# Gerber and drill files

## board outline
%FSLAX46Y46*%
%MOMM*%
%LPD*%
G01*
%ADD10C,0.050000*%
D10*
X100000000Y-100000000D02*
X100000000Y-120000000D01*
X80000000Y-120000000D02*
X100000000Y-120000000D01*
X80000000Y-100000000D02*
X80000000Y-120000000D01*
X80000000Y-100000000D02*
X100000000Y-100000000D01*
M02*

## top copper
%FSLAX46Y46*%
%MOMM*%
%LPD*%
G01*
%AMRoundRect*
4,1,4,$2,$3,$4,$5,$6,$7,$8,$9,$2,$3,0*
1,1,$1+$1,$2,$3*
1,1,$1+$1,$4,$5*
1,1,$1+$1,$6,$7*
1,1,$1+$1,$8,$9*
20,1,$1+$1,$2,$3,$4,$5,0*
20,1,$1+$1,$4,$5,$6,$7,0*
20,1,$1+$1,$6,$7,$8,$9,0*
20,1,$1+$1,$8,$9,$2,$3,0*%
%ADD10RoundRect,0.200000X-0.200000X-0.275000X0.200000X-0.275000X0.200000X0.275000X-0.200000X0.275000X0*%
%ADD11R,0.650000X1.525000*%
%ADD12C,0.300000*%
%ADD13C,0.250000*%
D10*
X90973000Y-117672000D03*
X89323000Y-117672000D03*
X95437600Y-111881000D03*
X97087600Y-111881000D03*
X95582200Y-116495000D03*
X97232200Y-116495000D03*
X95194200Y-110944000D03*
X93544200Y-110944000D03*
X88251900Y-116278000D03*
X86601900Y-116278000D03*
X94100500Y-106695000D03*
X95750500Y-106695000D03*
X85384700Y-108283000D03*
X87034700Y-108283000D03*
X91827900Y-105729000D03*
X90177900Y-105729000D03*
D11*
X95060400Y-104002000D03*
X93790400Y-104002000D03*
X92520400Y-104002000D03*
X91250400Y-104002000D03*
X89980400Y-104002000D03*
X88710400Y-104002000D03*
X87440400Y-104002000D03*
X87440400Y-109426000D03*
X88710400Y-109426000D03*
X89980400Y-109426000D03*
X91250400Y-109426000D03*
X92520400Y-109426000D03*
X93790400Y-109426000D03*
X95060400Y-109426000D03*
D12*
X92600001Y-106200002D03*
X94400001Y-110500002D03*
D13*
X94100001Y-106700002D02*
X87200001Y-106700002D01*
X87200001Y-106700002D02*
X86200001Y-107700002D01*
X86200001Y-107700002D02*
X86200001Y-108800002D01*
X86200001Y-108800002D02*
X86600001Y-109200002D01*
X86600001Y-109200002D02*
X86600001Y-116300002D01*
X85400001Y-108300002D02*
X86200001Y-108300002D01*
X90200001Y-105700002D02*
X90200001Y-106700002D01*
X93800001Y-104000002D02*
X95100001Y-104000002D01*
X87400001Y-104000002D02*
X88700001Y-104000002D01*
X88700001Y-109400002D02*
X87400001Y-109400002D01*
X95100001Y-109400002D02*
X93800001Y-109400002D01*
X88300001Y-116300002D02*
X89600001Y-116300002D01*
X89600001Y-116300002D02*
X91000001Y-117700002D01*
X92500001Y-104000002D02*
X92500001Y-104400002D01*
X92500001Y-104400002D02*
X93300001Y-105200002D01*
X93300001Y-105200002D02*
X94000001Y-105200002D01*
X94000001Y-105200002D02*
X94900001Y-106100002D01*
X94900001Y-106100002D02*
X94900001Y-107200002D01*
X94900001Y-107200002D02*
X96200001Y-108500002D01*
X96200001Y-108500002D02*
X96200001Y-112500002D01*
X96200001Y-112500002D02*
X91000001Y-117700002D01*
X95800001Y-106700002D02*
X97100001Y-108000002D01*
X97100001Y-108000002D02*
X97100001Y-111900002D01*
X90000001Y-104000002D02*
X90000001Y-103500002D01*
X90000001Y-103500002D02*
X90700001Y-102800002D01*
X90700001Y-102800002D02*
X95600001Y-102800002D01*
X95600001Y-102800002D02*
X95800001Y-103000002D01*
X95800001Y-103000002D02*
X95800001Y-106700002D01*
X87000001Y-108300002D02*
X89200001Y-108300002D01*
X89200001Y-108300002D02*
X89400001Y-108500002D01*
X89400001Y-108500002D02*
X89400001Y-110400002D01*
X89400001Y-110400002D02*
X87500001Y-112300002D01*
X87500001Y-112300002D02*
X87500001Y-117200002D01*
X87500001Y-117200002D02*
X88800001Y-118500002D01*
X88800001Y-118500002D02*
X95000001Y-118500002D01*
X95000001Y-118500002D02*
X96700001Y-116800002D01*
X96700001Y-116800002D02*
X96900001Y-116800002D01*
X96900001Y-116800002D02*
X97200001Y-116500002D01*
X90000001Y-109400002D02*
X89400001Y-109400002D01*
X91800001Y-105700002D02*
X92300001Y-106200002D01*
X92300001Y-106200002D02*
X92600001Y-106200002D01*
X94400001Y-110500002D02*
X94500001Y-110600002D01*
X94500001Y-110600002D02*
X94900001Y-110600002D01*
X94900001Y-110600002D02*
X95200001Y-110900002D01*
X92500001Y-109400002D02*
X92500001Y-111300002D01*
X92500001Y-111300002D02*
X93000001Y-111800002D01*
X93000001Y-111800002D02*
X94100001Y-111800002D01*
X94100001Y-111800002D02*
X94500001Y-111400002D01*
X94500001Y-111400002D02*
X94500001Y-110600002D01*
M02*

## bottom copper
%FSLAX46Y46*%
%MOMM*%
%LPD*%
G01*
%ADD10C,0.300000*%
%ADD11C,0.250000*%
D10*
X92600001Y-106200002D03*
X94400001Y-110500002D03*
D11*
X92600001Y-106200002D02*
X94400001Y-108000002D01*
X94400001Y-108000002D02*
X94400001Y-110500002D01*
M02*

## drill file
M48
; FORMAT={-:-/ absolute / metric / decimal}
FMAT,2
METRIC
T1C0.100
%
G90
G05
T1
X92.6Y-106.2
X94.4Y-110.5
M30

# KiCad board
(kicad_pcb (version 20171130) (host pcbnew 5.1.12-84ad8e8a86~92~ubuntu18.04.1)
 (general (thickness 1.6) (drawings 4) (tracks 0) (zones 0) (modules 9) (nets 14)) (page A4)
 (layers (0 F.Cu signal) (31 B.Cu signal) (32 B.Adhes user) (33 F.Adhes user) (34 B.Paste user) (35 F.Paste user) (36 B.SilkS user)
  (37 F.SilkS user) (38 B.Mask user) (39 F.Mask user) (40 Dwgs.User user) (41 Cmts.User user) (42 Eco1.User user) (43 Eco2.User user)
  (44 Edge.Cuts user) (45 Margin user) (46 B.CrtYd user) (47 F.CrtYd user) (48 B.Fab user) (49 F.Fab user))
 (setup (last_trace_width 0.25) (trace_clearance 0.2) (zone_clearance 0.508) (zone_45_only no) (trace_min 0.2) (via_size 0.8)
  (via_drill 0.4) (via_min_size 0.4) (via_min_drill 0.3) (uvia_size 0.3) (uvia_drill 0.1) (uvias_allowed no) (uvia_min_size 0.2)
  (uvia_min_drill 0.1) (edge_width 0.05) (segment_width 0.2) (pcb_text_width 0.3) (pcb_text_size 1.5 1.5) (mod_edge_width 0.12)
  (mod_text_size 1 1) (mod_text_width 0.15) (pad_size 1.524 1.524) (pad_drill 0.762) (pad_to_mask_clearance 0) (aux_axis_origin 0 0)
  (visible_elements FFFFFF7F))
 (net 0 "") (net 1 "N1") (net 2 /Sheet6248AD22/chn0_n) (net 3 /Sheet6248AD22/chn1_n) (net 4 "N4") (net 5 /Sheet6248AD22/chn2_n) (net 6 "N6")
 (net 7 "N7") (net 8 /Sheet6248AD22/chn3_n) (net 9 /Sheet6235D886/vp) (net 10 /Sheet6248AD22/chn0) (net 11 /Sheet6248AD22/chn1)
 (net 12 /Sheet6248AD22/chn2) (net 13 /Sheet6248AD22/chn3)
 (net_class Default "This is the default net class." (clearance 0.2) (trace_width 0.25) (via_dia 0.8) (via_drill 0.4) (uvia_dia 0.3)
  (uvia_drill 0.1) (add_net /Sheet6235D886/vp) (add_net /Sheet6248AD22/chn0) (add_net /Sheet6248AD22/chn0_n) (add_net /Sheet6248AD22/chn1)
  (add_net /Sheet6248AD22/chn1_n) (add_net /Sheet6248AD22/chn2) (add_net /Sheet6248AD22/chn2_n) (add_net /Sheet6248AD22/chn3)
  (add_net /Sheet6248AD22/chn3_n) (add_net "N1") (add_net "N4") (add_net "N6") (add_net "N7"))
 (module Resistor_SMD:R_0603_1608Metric (layer F.Cu) (at 90.148000 117.672000)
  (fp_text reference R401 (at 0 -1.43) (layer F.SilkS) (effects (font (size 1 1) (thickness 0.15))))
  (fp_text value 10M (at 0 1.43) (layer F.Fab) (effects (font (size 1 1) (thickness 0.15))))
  (pad 2 smd roundrect (at 0.825 0) (size 0.8 0.95) (layers F.Cu F.Mask F.Paste) (roundrect_rratio 0.25) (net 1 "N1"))
  (pad 1 smd roundrect (at -0.825 0) (size 0.8 0.95) (layers F.Cu F.Mask F.Paste) (roundrect_rratio 0.25) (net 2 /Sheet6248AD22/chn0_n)))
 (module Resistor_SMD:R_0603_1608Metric (layer F.Cu) (at 96.262600 111.881000)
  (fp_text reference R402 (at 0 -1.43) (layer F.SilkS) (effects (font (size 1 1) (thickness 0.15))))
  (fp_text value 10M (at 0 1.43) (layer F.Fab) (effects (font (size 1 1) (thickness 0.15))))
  (pad 1 smd roundrect (at -0.825 0) (size 0.8 0.95) (layers F.Cu F.Mask F.Paste) (roundrect_rratio 0.25) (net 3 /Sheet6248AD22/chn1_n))
  (pad 2 smd roundrect (at 0.825 0) (size 0.8 0.95) (layers F.Cu F.Mask F.Paste) (roundrect_rratio 0.25) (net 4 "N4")))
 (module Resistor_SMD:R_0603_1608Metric (layer F.Cu) (at 96.407200 116.495000)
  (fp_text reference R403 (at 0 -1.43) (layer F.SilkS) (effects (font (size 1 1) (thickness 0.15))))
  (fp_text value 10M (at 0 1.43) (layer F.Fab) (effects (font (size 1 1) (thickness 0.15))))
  (pad 1 smd roundrect (at -0.825 0) (size 0.8 0.95) (layers F.Cu F.Mask F.Paste) (roundrect_rratio 0.25) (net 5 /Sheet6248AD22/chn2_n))
  (pad 2 smd roundrect (at 0.825 0) (size 0.8 0.95) (layers F.Cu F.Mask F.Paste) (roundrect_rratio 0.25) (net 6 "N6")))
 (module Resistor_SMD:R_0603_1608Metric (layer F.Cu) (at 94.369200 110.944000)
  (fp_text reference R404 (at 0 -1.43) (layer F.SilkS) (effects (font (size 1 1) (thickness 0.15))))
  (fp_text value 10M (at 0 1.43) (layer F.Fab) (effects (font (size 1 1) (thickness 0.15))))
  (pad 2 smd roundrect (at 0.825 0) (size 0.8 0.95) (layers F.Cu F.Mask F.Paste) (roundrect_rratio 0.25) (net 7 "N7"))
  (pad 1 smd roundrect (at -0.825 0) (size 0.8 0.95) (layers F.Cu F.Mask F.Paste) (roundrect_rratio 0.25) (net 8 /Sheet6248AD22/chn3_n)))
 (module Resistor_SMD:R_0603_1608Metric (layer F.Cu) (at 87.426900 116.278000)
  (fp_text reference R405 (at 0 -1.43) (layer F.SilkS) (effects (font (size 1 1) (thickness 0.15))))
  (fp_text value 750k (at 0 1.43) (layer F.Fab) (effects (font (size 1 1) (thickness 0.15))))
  (pad 2 smd roundrect (at 0.825 0) (size 0.8 0.95) (layers F.Cu F.Mask F.Paste) (roundrect_rratio 0.25) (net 1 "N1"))
  (pad 1 smd roundrect (at -0.825 0) (size 0.8 0.95) (layers F.Cu F.Mask F.Paste) (roundrect_rratio 0.25) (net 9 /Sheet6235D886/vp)))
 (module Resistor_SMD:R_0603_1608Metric (layer F.Cu) (at 94.925500 106.695000)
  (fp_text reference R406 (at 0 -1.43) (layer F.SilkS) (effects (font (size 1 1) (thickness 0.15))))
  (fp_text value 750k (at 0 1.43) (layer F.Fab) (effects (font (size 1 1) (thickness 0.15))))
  (pad 1 smd roundrect (at -0.825 0) (size 0.8 0.95) (layers F.Cu F.Mask F.Paste) (roundrect_rratio 0.25) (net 9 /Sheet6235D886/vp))
  (pad 2 smd roundrect (at 0.825 0) (size 0.8 0.95) (layers F.Cu F.Mask F.Paste) (roundrect_rratio 0.25) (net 4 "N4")))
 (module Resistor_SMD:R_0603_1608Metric (layer F.Cu) (at 86.209700 108.283000)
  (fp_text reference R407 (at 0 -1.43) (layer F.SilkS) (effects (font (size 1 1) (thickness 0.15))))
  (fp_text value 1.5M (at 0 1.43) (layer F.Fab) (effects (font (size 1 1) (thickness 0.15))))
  (pad 1 smd roundrect (at -0.825 0) (size 0.8 0.95) (layers F.Cu F.Mask F.Paste) (roundrect_rratio 0.25) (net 9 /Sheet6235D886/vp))
  (pad 2 smd roundrect (at 0.825 0) (size 0.8 0.95) (layers F.Cu F.Mask F.Paste) (roundrect_rratio 0.25) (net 6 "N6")))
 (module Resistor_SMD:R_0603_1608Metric (layer F.Cu) (at 91.002900 105.729000)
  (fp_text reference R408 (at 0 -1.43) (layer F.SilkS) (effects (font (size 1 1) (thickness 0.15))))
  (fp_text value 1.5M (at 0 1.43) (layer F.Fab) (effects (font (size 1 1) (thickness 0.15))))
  (pad 2 smd roundrect (at 0.825 0) (size 0.8 0.95) (layers F.Cu F.Mask F.Paste) (roundrect_rratio 0.25) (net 7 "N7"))
  (pad 1 smd roundrect (at -0.825 0) (size 0.8 0.95) (layers F.Cu F.Mask F.Paste) (roundrect_rratio 0.25) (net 9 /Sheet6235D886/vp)))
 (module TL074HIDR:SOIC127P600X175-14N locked (layer F.Cu) (at 91.250400 106.714000 270.000000)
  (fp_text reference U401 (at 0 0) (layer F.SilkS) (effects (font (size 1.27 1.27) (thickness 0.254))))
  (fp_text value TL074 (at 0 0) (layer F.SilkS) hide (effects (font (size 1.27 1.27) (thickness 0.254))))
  (pad 1 smd rect (at -2.712 -3.81) (size 0.65 1.525) (layers F.Cu F.Mask F.Paste) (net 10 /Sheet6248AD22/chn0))
  (pad 2 smd rect (at -2.712 -2.54) (size 0.65 1.525) (layers F.Cu F.Mask F.Paste) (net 10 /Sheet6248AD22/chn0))
  (pad 3 smd rect (at -2.712 -1.27) (size 0.65 1.525) (layers F.Cu F.Mask F.Paste) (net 1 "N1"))
  (pad 4 smd rect (at -2.712 0) (size 0.65 1.525) (layers F.Cu F.Mask F.Paste))
  (pad 5 smd rect (at -2.712 1.27) (size 0.65 1.525) (layers F.Cu F.Mask F.Paste) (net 4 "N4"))
  (pad 6 smd rect (at -2.712 2.54) (size 0.65 1.525) (layers F.Cu F.Mask F.Paste) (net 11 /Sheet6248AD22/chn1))
  (pad 7 smd rect (at -2.712 3.81) (size 0.65 1.525) (layers F.Cu F.Mask F.Paste) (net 11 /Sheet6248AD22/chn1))
  (pad 8 smd rect (at 2.712 3.81) (size 0.65 1.525) (layers F.Cu F.Mask F.Paste) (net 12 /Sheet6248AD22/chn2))
  (pad 9 smd rect (at 2.712 2.54) (size 0.65 1.525) (layers F.Cu F.Mask F.Paste) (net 12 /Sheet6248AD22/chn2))
  (pad 10 smd rect (at 2.712 1.27) (size 0.65 1.525) (layers F.Cu F.Mask F.Paste) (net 6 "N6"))
  (pad 11 smd rect (at 2.712 0) (size 0.65 1.525) (layers F.Cu F.Mask F.Paste))
  (pad 12 smd rect (at 2.712 -1.27) (size 0.65 1.525) (layers F.Cu F.Mask F.Paste) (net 7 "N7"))
  (pad 13 smd rect (at 2.712 -2.54) (size 0.65 1.525) (layers F.Cu F.Mask F.Paste) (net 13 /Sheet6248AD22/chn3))
  (pad 14 smd rect (at 2.712 -3.81) (size 0.65 1.525) (layers F.Cu F.Mask F.Paste) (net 13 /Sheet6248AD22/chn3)))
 (gr_line (start 100 100) (end 100 120) (layer Edge.Cuts) (width 0.05))
 (gr_line (start 80 120) (end 100 120) (layer Edge.Cuts) (width 0.05))
 (gr_line (start 80 100) (end 80 120) (layer Edge.Cuts) (width 0.05))
 (gr_line (start 80 100) (end 100 100) (layer Edge.Cuts) (width 0.05))
 (segment (start 94.100001 106.700002) (end 87.200001 106.700002) (width 0.250000) (layer F.Cu) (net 9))
 (segment (start 87.200001 106.700002) (end 86.200001 107.700002) (width 0.250000) (layer F.Cu) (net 9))
 (segment (start 86.200001 107.700002) (end 86.200001 108.800002) (width 0.250000) (layer F.Cu) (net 9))
 (segment (start 86.200001 108.800002) (end 86.600001 109.200002) (width 0.250000) (layer F.Cu) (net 9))
 (segment (start 86.600001 109.200002) (end 86.600001 116.300002) (width 0.250000) (layer F.Cu) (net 9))
 (segment (start 85.400001 108.300002) (end 86.200001 108.300002) (width 0.250000) (layer F.Cu) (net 9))
 (segment (start 90.200001 105.700002) (end 90.200001 106.700002) (width 0.250000) (layer F.Cu) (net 9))
 (segment (start 93.800001 104.000002) (end 95.100001 104.000002) (width 0.250000) (layer F.Cu) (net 10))
 (segment (start 87.400001 104.000002) (end 88.700001 104.000002) (width 0.250000) (layer F.Cu) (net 11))
 (segment (start 88.700001 109.400002) (end 87.400001 109.400002) (width 0.250000) (layer F.Cu) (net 12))
 (segment (start 95.100001 109.400002) (end 93.800001 109.400002) (width 0.250000) (layer F.Cu) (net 13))
 (segment (start 88.300001 116.300002) (end 89.600001 116.300002) (width 0.250000) (layer F.Cu) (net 1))
 (segment (start 89.600001 116.300002) (end 91.000001 117.700002) (width 0.250000) (layer F.Cu) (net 1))
 (segment (start 92.500001 104.000002) (end 92.500001 104.400002) (width 0.250000) (layer F.Cu) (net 1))
 (segment (start 92.500001 104.400002) (end 93.300001 105.200002) (width 0.250000) (layer F.Cu) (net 1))
 (segment (start 93.300001 105.200002) (end 94.000001 105.200002) (width 0.250000) (layer F.Cu) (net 1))
 (segment (start 94.000001 105.200002) (end 94.900001 106.100002) (width 0.250000) (layer F.Cu) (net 1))
 (segment (start 94.900001 106.100002) (end 94.900001 107.200002) (width 0.250000) (layer F.Cu) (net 1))
 (segment (start 94.900001 107.200002) (end 96.200001 108.500002) (width 0.250000) (layer F.Cu) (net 1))
 (segment (start 96.200001 108.500002) (end 96.200001 112.500002) (width 0.250000) (layer F.Cu) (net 1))
 (segment (start 96.200001 112.500002) (end 91.000001 117.700002) (width 0.250000) (layer F.Cu) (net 1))
 (segment (start 95.800001 106.700002) (end 97.100001 108.000002) (width 0.250000) (layer F.Cu) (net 4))
 (segment (start 97.100001 108.000002) (end 97.100001 111.900002) (width 0.250000) (layer F.Cu) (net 4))
 (segment (start 90.000001 104.000002) (end 90.000001 103.500002) (width 0.250000) (layer F.Cu) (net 4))
 (segment (start 90.000001 103.500002) (end 90.700001 102.800002) (width 0.250000) (layer F.Cu) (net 4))
 (segment (start 90.700001 102.800002) (end 95.600001 102.800002) (width 0.250000) (layer F.Cu) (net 4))
 (segment (start 95.600001 102.800002) (end 95.800001 103.000002) (width 0.250000) (layer F.Cu) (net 4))
 (segment (start 95.800001 103.000002) (end 95.800001 106.700002) (width 0.250000) (layer F.Cu) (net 4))
 (segment (start 87.000001 108.300002) (end 89.200001 108.300002) (width 0.250000) (layer F.Cu) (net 6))
 (segment (start 89.200001 108.300002) (end 89.400001 108.500002) (width 0.250000) (layer F.Cu) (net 6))
 (segment (start 89.400001 108.500002) (end 89.400001 110.400002) (width 0.250000) (layer F.Cu) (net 6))
 (segment (start 89.400001 110.400002) (end 87.500001 112.300002) (width 0.250000) (layer F.Cu) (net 6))
 (segment (start 87.500001 112.300002) (end 87.500001 117.200002) (width 0.250000) (layer F.Cu) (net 6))
 (segment (start 87.500001 117.200002) (end 88.800001 118.500002) (width 0.250000) (layer F.Cu) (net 6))
 (segment (start 88.800001 118.500002) (end 95.000001 118.500002) (width 0.250000) (layer F.Cu) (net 6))
 (segment (start 95.000001 118.500002) (end 96.700001 116.800002) (width 0.250000) (layer F.Cu) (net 6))
 (segment (start 96.700001 116.800002) (end 96.900001 116.800002) (width 0.250000) (layer F.Cu) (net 6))
 (segment (start 96.900001 116.800002) (end 97.200001 116.500002) (width 0.250000) (layer F.Cu) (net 6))
 (segment (start 90.000001 109.400002) (end 89.400001 109.400002) (width 0.250000) (layer F.Cu) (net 6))
 (segment (start 91.800001 105.700002) (end 92.300001 106.200002) (width 0.250000) (layer F.Cu) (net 7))
 (segment (start 92.300001 106.200002) (end 92.600001 106.200002) (width 0.250000) (layer F.Cu) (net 7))
 (segment (start 92.600001 106.200002) (end 94.400001 108.000002) (width 0.250000) (layer B.Cu) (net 7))
 (segment (start 94.400001 108.000002) (end 94.400001 110.500002) (width 0.250000) (layer B.Cu) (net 7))
 (segment (start 94.400001 110.500002) (end 94.500001 110.600002) (width 0.250000) (layer F.Cu) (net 7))
 (segment (start 94.500001 110.600002) (end 94.900001 110.600002) (width 0.250000) (layer F.Cu) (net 7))
 (segment (start 94.900001 110.600002) (end 95.200001 110.900002) (width 0.250000) (layer F.Cu) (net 7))
 (segment (start 92.500001 109.400002) (end 92.500001 111.300002) (width 0.250000) (layer F.Cu) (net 7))
 (segment (start 92.500001 111.300002) (end 93.000001 111.800002) (width 0.250000) (layer F.Cu) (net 7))
 (segment (start 93.000001 111.800002) (end 94.100001 111.800002) (width 0.250000) (layer F.Cu) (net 7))
 (segment (start 94.100001 111.800002) (end 94.500001 111.400002) (width 0.250000) (layer F.Cu) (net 7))
 (segment (start 94.500001 111.400002) (end 94.500001 110.600002) (width 0.250000) (layer F.Cu) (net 7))
 (via micro (at 92.600001 106.200002) (size 0.300000) (drill 0.100000) (layers F.Cu B.Cu) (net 7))
 (via micro (at 94.400001 110.500002) (size 0.300000) (drill 0.100000) (layers F.Cu B.Cu) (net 7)))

